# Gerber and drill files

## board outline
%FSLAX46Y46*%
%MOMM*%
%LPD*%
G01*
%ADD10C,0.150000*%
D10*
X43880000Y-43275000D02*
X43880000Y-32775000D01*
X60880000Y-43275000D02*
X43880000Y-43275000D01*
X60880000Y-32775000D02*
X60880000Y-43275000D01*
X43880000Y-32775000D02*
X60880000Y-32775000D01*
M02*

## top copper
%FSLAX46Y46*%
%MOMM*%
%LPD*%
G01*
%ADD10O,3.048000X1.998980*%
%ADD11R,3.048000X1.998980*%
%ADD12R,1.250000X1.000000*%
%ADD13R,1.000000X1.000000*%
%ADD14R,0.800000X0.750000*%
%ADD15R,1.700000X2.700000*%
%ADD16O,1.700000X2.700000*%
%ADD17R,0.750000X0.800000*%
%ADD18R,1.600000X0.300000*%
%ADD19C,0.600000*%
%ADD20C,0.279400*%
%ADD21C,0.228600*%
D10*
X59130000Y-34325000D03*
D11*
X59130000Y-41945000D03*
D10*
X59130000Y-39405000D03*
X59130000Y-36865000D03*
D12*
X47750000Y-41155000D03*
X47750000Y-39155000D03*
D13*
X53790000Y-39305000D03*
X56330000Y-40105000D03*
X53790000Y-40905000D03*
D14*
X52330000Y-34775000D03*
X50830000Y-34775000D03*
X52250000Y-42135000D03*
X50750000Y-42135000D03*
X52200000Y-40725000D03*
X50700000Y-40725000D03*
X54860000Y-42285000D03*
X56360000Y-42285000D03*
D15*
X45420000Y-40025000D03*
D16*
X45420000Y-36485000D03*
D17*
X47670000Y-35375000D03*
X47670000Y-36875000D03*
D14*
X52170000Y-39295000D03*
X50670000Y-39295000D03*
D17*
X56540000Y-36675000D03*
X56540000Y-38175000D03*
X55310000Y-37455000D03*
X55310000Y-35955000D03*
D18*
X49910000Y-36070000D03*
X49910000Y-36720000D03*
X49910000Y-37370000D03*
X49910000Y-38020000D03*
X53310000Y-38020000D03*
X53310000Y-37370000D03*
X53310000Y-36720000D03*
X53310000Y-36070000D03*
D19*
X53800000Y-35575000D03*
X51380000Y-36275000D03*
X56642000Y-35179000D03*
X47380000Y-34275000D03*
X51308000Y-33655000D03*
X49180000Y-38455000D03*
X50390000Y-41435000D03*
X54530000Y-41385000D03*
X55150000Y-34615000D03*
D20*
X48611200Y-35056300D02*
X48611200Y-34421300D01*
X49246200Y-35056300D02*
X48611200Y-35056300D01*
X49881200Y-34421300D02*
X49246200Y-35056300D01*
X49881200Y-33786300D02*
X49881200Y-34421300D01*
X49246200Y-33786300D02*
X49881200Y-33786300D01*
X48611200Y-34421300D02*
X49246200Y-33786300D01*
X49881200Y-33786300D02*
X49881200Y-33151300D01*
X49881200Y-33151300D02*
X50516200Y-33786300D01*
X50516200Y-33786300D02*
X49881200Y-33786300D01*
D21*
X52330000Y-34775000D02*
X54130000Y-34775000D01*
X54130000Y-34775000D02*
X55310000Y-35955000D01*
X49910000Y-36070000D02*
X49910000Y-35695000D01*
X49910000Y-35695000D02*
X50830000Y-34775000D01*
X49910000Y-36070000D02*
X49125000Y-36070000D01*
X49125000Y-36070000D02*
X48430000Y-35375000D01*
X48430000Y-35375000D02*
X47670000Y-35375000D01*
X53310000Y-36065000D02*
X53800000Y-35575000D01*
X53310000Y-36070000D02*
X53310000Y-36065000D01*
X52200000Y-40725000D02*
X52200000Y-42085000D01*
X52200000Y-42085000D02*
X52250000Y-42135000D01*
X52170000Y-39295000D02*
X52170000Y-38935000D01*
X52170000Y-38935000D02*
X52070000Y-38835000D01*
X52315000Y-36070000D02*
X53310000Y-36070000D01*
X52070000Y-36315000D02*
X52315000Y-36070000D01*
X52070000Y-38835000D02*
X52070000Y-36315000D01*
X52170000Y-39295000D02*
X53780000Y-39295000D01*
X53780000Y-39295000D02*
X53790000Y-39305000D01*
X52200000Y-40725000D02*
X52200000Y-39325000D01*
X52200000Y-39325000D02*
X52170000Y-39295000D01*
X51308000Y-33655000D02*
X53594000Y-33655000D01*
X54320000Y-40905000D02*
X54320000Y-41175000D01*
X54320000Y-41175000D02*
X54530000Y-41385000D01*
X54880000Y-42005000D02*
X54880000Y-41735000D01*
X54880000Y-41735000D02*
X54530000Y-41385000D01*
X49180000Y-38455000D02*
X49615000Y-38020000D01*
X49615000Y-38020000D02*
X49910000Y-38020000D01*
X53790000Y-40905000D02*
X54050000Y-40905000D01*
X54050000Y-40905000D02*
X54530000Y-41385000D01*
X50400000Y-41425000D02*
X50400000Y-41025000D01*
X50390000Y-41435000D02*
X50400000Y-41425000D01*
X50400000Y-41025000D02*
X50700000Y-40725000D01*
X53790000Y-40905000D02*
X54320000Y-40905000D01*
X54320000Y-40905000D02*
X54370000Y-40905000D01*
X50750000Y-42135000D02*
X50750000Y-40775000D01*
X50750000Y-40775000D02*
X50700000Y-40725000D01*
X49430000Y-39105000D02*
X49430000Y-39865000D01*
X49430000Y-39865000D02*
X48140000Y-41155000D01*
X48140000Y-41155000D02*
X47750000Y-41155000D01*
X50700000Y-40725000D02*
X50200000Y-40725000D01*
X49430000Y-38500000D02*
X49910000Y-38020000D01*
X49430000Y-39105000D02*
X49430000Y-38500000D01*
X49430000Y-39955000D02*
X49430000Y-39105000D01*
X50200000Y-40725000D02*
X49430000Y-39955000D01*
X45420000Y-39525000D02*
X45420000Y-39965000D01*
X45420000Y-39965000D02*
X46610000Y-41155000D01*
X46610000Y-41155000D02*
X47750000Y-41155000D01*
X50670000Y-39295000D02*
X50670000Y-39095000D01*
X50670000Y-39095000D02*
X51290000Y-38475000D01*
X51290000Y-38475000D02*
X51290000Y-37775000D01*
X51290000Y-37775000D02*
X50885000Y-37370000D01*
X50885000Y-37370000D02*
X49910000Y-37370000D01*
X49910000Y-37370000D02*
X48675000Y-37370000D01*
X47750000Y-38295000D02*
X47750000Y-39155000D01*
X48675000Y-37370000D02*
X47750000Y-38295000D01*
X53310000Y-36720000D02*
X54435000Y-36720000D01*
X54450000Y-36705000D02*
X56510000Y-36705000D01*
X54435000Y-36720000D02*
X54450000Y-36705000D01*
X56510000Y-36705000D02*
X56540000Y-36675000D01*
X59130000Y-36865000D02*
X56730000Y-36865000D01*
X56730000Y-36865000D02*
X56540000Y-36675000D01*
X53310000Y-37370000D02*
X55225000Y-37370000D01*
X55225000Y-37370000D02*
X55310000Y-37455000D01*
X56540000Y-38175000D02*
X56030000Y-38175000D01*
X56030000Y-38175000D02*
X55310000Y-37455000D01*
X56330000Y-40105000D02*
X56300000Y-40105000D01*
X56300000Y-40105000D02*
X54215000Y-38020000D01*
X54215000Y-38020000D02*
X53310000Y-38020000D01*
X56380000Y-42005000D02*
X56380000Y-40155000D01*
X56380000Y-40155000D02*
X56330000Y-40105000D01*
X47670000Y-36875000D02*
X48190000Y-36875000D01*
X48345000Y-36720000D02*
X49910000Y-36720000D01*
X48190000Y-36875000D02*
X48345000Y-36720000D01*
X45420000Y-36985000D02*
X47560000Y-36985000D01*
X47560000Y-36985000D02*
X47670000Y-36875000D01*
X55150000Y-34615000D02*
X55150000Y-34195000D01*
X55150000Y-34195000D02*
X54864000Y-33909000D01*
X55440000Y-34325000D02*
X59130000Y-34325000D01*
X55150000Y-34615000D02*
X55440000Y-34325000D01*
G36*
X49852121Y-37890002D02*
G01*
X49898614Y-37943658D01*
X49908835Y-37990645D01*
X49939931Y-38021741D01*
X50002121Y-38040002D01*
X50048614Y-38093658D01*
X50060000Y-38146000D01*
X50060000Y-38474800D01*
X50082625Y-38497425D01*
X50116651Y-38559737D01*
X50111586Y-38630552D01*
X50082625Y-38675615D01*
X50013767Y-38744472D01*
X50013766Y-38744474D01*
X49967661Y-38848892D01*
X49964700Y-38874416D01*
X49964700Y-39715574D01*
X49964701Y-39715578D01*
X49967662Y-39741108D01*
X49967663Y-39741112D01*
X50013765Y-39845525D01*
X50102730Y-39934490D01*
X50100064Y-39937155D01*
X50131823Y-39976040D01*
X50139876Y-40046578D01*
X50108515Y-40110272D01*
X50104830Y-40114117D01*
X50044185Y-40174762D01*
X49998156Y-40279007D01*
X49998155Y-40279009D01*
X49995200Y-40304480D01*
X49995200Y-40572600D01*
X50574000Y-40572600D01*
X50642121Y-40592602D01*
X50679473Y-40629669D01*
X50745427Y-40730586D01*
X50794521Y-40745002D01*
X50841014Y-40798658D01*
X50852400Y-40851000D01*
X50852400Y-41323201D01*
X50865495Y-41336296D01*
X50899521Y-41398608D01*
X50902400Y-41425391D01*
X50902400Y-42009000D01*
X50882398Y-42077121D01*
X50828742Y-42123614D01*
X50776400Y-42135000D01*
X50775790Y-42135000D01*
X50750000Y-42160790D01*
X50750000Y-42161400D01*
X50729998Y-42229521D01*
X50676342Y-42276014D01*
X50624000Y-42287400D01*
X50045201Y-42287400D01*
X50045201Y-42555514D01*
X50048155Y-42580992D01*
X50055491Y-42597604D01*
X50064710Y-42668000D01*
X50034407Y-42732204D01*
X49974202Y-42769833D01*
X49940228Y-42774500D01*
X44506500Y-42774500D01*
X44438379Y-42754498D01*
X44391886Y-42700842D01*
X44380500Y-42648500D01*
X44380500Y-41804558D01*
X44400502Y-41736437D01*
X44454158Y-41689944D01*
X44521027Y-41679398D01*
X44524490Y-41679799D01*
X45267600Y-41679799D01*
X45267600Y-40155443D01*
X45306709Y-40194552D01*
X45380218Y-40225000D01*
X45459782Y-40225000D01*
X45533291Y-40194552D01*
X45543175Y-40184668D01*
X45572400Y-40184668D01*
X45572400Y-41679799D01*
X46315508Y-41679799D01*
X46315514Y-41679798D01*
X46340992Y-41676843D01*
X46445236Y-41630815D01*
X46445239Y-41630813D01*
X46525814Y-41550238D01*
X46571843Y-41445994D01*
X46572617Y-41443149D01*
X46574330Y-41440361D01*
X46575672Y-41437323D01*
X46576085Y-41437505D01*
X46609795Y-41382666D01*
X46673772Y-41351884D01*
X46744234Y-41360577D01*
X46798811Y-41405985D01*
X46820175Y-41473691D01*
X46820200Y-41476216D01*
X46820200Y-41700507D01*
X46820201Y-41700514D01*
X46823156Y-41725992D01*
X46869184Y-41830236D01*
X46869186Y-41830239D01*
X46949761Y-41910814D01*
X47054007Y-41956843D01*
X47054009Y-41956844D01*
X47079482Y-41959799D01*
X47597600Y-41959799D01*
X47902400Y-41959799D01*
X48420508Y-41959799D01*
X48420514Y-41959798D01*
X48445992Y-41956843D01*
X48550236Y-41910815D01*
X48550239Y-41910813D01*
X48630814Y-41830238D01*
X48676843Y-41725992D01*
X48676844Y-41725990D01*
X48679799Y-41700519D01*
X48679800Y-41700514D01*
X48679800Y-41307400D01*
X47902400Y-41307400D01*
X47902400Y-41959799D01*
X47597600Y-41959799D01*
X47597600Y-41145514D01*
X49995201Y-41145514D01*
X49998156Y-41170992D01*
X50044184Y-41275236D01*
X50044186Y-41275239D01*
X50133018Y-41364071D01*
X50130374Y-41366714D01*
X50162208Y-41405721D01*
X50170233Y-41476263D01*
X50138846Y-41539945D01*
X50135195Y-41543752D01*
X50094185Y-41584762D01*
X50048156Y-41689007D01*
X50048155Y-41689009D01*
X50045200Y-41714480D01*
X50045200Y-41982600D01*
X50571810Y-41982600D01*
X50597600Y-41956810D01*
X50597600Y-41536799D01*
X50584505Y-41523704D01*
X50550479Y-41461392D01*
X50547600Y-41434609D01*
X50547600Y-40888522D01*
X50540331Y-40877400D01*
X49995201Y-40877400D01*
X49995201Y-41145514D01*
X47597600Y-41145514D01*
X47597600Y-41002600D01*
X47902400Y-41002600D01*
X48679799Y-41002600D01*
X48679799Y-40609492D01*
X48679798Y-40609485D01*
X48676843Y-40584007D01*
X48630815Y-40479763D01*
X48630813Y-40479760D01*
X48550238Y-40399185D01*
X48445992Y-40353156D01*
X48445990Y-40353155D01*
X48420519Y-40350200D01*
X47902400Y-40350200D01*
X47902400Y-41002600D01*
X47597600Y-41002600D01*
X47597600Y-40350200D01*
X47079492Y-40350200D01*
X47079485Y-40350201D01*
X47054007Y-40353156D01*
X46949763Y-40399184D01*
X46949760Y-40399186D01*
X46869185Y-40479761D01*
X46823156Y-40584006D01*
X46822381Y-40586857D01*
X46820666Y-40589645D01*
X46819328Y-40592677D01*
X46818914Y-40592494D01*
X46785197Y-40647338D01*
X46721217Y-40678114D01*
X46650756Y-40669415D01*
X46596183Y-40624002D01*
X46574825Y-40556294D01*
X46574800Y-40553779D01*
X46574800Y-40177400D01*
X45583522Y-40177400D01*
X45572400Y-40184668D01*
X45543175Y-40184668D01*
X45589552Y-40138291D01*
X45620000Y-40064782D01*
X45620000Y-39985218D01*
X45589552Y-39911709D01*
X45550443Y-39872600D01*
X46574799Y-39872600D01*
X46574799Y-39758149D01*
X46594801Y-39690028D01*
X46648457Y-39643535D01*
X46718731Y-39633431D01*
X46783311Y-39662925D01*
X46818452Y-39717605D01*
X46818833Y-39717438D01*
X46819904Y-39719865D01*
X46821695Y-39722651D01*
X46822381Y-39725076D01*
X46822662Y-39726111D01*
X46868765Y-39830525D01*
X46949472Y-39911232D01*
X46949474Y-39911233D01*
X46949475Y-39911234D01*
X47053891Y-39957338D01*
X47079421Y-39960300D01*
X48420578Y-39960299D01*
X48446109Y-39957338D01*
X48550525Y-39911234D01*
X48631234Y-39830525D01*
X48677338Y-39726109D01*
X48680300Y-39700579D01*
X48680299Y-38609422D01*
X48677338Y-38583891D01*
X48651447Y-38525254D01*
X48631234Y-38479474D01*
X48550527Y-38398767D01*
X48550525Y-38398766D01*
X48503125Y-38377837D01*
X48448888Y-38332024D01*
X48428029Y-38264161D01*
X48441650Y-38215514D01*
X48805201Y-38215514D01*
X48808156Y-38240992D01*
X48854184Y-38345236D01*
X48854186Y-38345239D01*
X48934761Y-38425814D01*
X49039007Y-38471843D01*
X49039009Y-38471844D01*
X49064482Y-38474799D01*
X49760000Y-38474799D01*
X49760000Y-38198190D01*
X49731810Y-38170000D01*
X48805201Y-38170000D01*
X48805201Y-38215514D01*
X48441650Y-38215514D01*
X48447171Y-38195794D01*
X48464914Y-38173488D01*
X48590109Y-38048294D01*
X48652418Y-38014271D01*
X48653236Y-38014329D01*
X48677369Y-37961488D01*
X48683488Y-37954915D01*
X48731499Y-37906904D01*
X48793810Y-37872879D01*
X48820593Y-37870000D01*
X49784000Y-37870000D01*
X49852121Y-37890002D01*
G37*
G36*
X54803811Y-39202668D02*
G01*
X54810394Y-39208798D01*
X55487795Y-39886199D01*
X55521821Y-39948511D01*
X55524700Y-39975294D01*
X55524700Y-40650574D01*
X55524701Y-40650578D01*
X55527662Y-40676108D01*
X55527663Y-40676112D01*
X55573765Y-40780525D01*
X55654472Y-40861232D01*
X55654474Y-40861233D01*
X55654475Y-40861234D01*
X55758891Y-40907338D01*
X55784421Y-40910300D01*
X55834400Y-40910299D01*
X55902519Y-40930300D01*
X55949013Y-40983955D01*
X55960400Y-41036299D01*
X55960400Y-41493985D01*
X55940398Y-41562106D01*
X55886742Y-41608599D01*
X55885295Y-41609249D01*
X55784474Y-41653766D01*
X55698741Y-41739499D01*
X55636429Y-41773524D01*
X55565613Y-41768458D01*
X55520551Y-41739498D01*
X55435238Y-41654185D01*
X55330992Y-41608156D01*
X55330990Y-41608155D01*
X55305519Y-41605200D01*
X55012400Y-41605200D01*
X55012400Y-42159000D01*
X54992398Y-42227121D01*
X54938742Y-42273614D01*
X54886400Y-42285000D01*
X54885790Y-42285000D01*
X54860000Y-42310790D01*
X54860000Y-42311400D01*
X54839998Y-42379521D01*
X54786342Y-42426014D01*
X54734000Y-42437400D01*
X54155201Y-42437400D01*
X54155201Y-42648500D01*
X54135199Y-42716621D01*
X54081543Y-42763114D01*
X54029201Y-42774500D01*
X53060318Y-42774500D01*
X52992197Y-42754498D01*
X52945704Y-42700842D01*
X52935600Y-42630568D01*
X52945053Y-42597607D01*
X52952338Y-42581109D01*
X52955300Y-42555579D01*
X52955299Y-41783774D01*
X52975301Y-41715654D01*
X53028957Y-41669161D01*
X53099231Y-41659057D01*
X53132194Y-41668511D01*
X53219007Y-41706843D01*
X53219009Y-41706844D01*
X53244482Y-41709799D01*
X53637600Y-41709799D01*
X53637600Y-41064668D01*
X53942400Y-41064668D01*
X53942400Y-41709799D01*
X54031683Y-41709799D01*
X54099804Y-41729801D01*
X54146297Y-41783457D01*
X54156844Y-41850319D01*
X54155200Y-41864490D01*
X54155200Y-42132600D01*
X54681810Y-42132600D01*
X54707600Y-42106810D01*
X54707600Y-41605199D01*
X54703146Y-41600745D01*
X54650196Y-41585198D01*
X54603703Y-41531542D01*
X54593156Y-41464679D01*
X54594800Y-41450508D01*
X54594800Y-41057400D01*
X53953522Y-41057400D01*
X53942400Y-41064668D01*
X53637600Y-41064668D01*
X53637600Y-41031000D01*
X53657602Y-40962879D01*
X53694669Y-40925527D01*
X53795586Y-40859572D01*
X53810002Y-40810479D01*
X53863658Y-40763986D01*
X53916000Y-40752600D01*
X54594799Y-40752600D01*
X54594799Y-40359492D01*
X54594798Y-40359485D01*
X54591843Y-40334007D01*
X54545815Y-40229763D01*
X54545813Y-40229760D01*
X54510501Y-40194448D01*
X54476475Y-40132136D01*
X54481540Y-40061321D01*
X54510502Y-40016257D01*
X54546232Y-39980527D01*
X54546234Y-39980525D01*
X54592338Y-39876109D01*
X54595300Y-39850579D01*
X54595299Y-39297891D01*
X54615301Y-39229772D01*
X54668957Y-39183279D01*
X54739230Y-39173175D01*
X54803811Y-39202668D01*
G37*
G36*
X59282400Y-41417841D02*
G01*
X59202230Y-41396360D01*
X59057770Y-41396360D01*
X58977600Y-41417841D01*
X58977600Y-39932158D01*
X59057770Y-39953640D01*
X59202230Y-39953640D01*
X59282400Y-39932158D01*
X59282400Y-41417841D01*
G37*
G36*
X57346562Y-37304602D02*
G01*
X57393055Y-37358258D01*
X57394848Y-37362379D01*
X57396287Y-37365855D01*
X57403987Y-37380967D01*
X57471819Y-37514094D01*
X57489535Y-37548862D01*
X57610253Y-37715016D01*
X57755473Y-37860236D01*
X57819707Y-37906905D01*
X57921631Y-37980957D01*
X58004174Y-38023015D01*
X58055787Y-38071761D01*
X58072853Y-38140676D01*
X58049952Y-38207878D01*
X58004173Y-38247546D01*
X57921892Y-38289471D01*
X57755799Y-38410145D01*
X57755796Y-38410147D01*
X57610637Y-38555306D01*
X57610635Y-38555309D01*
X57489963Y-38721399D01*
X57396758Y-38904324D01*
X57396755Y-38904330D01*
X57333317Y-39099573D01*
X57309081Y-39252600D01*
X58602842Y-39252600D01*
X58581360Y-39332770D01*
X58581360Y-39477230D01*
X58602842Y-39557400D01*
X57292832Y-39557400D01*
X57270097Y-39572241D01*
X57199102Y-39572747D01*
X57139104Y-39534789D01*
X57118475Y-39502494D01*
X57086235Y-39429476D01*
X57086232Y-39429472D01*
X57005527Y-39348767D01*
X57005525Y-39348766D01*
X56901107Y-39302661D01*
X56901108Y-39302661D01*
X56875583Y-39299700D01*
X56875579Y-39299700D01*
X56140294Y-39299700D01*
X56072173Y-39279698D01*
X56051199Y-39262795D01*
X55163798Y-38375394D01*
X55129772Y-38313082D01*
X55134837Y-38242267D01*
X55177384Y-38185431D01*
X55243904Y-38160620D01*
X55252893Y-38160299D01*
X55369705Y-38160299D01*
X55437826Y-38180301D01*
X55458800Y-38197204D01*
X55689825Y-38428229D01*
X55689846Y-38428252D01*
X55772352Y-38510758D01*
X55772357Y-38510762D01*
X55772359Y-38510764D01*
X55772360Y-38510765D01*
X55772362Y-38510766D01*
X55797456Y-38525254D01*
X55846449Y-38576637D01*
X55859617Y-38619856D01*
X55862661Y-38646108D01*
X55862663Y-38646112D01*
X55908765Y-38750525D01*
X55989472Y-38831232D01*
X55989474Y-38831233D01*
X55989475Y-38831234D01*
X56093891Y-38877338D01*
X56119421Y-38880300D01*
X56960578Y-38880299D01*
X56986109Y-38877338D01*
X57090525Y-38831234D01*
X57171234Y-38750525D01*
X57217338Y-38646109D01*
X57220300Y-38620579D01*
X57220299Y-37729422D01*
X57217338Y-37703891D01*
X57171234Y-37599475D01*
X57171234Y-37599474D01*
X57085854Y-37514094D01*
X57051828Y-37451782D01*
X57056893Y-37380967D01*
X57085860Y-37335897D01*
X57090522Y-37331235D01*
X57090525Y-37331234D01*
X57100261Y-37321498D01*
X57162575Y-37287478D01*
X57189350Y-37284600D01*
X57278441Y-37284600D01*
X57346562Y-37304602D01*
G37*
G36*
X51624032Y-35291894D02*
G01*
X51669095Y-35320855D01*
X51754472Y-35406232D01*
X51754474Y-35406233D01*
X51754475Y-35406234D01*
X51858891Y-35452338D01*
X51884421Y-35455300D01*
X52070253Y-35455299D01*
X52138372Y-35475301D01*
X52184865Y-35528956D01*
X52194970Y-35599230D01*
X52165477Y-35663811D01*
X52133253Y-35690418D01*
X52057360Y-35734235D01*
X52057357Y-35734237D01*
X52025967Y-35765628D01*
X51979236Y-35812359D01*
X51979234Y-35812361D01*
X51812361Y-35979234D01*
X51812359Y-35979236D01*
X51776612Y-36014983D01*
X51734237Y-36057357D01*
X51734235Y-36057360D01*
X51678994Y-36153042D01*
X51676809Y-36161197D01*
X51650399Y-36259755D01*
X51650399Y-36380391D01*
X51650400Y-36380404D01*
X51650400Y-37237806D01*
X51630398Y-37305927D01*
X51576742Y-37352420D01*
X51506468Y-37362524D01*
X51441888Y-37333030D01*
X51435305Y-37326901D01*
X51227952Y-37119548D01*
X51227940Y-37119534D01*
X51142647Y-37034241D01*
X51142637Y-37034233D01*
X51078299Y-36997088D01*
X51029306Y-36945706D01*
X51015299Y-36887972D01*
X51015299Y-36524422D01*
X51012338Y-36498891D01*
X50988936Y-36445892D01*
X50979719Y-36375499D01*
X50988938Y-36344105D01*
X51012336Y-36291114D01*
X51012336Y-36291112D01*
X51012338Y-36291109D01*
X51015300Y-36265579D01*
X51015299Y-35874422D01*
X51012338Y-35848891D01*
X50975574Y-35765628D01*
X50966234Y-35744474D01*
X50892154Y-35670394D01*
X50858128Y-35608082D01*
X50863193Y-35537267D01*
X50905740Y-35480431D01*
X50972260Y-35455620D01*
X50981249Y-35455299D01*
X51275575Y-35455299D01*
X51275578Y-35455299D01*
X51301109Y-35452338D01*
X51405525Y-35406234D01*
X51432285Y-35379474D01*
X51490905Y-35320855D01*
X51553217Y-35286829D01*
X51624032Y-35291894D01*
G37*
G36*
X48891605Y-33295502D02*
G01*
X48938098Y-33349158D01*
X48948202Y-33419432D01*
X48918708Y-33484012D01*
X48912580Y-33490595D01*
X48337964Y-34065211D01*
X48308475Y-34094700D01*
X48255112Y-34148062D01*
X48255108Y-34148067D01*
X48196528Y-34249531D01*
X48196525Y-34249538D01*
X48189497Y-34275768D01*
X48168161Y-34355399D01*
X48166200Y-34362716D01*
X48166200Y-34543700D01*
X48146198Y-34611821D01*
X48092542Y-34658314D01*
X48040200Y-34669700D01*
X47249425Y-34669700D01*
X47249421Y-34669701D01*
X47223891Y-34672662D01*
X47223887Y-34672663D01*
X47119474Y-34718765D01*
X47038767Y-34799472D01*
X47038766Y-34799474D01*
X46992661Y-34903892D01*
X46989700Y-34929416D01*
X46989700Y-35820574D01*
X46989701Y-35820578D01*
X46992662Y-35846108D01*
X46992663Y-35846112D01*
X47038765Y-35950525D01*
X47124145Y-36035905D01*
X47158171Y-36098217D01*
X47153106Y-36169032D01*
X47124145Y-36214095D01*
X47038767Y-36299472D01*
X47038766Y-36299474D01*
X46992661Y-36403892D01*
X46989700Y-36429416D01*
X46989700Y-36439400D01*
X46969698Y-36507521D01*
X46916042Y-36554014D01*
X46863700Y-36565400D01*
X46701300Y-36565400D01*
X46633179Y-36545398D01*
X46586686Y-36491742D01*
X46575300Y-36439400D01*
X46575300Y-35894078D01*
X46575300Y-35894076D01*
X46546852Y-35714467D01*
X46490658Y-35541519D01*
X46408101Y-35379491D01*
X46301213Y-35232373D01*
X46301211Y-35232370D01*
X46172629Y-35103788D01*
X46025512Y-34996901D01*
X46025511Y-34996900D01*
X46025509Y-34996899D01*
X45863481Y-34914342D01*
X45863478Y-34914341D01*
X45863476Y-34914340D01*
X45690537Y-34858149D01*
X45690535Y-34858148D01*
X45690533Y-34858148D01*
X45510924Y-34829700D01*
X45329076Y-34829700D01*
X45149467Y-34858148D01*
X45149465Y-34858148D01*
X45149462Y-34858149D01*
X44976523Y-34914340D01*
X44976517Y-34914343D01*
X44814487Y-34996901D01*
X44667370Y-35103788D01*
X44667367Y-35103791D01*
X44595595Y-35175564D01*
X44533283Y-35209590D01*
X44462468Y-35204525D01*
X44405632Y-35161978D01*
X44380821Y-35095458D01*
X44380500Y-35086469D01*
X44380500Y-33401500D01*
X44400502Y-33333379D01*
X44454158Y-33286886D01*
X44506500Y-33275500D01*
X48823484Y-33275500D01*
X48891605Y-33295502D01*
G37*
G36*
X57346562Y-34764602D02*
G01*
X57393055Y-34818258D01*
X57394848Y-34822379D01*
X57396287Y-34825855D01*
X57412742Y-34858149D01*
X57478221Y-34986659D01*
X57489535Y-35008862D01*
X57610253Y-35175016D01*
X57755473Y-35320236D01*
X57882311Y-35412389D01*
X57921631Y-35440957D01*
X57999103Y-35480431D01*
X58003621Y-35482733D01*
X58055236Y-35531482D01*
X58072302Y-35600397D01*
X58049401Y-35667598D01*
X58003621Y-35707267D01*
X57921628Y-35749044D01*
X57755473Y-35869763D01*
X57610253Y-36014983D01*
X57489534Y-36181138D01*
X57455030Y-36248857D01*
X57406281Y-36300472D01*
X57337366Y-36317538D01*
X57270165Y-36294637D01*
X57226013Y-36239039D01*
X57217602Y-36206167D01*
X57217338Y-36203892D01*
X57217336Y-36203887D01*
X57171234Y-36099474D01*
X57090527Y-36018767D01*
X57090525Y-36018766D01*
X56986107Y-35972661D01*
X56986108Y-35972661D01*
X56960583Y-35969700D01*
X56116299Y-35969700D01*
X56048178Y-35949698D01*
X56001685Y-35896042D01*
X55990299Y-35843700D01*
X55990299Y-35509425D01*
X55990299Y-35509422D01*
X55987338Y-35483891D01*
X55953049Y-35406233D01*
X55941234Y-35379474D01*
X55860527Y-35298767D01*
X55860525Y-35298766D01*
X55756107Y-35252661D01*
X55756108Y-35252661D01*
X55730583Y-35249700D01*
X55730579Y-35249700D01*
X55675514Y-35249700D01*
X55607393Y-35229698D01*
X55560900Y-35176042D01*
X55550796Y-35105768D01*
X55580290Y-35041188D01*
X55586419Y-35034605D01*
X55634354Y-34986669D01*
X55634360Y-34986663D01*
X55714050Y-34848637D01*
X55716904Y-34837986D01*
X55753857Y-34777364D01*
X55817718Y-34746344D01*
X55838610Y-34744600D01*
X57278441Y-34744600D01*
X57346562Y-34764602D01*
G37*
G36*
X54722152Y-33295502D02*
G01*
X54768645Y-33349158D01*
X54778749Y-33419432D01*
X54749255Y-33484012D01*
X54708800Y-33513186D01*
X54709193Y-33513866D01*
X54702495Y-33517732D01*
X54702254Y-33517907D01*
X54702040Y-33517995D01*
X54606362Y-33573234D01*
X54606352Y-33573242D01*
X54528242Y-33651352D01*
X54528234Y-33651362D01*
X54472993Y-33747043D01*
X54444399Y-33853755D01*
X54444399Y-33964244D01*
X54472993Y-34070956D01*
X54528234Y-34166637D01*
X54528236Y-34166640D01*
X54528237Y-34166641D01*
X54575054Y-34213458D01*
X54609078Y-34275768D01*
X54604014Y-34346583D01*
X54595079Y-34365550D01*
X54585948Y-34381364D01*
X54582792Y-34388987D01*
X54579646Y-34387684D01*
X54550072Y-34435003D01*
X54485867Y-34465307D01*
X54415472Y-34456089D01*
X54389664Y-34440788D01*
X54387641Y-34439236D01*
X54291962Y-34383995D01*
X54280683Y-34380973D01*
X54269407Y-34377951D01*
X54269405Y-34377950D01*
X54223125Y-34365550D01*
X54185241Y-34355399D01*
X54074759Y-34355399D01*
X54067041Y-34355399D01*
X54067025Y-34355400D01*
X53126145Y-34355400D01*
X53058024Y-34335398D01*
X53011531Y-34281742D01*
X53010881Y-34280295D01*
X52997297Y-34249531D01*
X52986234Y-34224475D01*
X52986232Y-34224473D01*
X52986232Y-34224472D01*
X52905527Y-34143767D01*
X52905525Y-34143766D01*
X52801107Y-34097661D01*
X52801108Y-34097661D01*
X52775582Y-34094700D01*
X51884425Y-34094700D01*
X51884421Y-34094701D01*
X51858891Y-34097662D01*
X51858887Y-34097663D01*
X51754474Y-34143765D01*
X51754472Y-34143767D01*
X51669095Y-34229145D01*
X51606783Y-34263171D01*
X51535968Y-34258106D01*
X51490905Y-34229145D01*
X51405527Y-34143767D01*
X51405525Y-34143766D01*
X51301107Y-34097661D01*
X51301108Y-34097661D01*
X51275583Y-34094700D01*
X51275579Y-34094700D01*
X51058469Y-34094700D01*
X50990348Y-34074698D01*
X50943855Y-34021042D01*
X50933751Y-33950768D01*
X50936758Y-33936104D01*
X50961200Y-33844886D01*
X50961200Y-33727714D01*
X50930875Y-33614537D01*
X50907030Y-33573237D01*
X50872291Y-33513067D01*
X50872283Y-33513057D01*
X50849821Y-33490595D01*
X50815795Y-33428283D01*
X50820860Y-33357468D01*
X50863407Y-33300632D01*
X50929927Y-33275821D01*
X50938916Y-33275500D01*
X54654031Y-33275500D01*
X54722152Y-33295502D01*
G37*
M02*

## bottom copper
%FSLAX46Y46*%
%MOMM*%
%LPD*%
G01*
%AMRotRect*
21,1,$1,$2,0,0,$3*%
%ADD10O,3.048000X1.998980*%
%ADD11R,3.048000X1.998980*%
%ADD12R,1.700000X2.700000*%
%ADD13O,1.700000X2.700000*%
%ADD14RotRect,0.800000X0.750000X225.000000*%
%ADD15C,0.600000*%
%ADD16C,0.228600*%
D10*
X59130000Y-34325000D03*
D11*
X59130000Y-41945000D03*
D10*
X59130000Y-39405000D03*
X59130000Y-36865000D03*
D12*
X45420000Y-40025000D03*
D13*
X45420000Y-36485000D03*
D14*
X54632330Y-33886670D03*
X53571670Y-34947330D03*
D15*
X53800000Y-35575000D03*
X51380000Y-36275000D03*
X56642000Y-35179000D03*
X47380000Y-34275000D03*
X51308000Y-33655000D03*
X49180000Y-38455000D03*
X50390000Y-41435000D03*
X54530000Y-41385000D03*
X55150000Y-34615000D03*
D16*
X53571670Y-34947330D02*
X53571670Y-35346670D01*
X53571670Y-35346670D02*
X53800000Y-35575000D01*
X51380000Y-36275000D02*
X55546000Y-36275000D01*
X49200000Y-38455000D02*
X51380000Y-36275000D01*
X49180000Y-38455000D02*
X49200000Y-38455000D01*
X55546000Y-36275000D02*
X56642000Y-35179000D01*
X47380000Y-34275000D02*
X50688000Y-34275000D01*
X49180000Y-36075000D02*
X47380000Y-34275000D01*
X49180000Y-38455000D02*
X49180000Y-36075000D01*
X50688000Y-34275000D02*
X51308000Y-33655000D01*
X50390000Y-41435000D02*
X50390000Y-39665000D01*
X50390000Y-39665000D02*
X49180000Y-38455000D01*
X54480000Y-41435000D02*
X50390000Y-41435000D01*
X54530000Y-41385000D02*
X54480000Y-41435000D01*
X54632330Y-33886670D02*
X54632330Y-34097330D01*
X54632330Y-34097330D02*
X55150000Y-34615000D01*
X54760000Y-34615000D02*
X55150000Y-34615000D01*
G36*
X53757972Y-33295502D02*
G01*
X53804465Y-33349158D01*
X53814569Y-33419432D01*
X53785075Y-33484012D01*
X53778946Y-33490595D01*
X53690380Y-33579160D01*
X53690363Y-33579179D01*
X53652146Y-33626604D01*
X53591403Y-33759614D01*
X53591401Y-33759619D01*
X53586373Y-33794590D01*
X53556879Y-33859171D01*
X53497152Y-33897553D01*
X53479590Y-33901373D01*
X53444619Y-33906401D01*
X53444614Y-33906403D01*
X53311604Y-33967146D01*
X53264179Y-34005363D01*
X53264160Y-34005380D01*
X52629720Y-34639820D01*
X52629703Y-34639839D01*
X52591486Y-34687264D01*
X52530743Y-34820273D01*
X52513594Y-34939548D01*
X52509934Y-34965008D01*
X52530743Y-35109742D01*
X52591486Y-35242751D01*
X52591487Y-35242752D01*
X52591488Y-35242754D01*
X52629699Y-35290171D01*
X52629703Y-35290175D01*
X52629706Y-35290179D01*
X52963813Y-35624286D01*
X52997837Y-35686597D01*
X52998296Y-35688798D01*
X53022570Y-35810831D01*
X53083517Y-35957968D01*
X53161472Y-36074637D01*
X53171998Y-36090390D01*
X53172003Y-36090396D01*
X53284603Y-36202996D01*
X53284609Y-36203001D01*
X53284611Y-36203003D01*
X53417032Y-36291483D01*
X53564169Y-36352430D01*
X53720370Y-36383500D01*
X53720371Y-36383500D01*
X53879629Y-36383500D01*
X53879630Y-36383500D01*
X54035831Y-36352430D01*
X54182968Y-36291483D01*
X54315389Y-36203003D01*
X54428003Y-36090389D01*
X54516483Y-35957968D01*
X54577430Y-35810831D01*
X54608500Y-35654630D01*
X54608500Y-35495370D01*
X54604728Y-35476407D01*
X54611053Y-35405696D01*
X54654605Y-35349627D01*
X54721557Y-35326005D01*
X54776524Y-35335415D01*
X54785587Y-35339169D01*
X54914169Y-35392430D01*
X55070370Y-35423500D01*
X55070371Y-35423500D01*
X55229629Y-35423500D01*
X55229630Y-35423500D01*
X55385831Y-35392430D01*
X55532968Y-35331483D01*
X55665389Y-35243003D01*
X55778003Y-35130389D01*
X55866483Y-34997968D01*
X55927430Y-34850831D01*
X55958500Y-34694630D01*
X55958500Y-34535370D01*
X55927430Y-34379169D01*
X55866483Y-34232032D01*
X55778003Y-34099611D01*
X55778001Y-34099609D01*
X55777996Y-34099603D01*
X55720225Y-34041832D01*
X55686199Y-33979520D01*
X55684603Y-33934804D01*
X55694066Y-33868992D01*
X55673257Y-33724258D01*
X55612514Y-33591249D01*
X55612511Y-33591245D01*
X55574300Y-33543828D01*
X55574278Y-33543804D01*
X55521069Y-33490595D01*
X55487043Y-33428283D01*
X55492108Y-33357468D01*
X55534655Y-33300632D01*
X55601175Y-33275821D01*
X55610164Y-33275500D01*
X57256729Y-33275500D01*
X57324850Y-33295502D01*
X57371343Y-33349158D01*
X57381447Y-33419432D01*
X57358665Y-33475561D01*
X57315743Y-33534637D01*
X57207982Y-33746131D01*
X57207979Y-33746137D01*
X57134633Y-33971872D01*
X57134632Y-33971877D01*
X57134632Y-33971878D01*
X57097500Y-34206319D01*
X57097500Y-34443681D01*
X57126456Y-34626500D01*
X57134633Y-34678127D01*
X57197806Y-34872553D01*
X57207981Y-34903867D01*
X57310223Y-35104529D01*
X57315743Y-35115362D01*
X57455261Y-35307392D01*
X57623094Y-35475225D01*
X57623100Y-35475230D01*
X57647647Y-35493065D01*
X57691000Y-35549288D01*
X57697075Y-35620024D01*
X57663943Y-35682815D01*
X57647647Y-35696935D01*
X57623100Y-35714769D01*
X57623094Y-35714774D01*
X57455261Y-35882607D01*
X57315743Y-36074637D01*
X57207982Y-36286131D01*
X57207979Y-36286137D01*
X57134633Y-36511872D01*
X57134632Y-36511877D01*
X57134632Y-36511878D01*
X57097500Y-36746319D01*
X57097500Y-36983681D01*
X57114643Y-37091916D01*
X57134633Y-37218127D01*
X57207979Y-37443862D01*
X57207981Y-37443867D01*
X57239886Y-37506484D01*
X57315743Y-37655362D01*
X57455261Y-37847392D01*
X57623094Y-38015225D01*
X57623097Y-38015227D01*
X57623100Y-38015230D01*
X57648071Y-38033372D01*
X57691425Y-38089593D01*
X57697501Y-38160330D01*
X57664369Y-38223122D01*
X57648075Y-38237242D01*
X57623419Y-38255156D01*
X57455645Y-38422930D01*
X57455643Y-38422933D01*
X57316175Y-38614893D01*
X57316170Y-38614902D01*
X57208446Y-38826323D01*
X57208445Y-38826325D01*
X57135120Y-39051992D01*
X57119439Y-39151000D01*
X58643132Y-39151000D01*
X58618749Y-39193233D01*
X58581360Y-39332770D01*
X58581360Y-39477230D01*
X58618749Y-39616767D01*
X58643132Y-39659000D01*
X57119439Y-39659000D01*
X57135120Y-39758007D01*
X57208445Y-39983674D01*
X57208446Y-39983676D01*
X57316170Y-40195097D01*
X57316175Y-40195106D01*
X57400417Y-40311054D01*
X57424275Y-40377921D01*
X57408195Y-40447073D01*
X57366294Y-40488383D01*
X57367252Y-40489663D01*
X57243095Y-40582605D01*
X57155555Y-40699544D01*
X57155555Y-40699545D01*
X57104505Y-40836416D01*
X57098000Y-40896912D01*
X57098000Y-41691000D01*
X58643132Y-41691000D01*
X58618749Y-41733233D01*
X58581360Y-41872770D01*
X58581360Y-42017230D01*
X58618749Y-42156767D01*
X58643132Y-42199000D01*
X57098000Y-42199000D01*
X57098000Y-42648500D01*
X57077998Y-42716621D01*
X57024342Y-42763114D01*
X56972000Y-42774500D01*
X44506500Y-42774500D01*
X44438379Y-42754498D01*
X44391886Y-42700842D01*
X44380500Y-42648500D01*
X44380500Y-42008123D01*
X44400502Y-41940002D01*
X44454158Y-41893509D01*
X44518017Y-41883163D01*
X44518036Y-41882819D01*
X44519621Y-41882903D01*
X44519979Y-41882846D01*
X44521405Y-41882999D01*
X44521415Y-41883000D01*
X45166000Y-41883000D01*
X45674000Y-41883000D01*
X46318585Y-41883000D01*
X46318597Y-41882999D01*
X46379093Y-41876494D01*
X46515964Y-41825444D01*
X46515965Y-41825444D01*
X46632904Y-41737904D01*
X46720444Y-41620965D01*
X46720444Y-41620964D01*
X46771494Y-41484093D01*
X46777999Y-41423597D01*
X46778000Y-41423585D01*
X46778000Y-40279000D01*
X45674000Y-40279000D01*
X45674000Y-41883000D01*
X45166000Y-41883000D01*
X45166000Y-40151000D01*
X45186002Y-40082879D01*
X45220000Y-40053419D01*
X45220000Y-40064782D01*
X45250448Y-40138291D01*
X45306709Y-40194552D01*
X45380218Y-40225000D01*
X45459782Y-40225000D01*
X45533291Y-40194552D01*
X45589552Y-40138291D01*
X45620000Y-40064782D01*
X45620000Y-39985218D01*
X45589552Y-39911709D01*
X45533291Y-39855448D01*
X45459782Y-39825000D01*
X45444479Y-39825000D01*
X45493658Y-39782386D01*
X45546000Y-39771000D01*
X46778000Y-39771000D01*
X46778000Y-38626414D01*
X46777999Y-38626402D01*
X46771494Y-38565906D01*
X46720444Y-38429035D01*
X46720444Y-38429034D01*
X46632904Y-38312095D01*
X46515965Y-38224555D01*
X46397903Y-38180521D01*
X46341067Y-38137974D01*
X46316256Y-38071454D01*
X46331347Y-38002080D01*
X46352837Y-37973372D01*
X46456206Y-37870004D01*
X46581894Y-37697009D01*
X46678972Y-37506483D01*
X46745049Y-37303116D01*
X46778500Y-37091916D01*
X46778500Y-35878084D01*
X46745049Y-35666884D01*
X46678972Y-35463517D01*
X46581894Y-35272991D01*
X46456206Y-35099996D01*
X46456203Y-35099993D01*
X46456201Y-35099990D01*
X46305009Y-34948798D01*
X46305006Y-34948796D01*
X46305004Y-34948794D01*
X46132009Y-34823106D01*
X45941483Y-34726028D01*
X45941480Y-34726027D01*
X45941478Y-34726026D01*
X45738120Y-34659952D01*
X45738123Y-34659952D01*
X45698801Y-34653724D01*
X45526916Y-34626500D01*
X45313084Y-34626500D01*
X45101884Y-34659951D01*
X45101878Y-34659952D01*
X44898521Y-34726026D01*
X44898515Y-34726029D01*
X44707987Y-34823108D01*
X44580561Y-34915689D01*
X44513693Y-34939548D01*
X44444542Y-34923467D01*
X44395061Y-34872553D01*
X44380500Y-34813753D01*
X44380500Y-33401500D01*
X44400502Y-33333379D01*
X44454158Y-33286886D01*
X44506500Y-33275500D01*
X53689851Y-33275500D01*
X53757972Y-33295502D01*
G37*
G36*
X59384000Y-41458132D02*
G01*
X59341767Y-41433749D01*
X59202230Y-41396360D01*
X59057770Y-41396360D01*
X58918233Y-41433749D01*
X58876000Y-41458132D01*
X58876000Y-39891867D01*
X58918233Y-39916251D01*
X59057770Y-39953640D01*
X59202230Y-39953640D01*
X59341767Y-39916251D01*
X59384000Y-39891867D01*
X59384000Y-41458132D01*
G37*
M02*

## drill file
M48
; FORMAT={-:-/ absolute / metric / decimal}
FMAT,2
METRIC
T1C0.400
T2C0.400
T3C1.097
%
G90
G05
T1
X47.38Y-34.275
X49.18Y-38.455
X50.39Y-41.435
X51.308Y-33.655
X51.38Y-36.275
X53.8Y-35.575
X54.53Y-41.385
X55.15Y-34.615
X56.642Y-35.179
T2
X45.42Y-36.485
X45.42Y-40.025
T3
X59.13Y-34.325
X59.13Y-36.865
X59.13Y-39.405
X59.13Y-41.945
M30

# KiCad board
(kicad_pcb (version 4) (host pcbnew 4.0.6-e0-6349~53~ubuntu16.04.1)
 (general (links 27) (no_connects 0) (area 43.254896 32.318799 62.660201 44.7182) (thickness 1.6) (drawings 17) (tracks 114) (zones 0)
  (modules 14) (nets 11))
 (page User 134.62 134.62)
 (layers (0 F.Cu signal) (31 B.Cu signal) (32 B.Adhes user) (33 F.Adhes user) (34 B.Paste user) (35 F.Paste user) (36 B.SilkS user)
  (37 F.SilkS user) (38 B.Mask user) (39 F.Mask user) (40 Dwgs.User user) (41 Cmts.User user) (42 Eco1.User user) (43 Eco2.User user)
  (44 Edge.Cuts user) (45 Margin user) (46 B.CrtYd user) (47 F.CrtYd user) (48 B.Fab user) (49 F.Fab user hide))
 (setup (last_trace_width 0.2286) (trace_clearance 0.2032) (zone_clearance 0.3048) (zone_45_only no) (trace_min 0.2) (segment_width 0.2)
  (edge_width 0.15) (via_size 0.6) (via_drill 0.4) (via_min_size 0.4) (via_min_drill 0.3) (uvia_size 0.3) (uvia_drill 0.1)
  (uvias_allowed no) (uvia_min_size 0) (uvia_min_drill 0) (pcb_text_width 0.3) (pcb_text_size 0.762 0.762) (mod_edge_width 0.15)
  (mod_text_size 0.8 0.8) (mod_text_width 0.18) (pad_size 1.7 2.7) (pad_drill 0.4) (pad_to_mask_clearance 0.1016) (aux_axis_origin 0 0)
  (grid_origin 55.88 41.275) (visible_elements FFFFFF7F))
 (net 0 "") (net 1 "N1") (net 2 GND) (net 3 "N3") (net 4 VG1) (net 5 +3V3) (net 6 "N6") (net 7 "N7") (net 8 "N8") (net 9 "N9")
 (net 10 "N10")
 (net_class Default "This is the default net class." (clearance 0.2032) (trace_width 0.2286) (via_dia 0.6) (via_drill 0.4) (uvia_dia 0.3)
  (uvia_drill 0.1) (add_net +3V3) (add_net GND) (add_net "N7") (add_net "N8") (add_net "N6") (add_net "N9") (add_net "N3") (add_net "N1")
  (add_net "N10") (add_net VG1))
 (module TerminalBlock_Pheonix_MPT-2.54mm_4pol (layer F.Cu) (at 59.13 41.945 90)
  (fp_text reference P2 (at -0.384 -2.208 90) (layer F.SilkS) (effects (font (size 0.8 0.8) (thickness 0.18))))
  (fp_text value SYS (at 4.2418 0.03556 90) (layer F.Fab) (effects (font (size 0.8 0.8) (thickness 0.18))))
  (pad 4 thru_hole oval (at 7.62 0 270) (size 1.99898 3.048) (drill 1.09728) (layers *.Cu *.Mask F.SilkS) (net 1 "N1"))
  (pad 1 thru_hole rect (at 0 0 270) (size 1.99898 3.048) (drill 1.09728) (layers *.Cu *.Mask F.SilkS) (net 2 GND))
  (pad 2 thru_hole oval (at 2.54 0 270) (size 1.99898 3.048) (drill 1.09728) (layers *.Cu *.Mask F.SilkS) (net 2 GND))
  (pad 3 thru_hole oval (at 5.08 0 270) (size 1.99898 3.048) (drill 1.09728) (layers *.Cu *.Mask F.SilkS) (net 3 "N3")))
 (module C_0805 (layer F.Cu) (at 47.75 40.155 90)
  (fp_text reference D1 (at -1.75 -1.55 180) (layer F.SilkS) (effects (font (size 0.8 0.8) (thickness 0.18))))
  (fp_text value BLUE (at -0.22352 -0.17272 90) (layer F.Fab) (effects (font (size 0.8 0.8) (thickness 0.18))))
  (pad 1 smd rect (at -1 0 90) (size 1 1.25) (layers F.Cu F.Paste F.Mask) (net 2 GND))
  (pad 2 smd rect (at 1 0 90) (size 1 1.25) (layers F.Cu F.Paste F.Mask) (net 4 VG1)))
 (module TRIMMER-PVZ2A (layer F.Cu) (at 53.79 40.105 270)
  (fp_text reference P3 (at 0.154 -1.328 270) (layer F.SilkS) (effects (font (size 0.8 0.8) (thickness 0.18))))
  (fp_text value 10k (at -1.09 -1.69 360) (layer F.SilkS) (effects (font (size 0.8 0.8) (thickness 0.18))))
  (pad 1 smd rect (at -0.8 0 270) (size 1 1) (layers F.Cu F.Paste F.Mask) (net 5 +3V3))
  (pad 2 smd rect (at 0 -2.54 270) (size 1 1) (layers F.Cu F.Paste F.Mask) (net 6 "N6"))
  (pad 3 smd rect (at 0.8 0 270) (size 1 1) (layers F.Cu F.Paste F.Mask) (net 2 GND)))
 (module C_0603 (layer F.Cu) (at 51.58 34.775 180)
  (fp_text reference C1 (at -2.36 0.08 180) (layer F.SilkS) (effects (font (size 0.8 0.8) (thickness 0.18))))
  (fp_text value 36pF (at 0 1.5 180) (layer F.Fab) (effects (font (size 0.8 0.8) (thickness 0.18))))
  (pad 1 smd rect (at -0.75 0 180) (size 0.8 0.75) (layers F.Cu F.Paste F.Mask) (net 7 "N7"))
  (pad 2 smd rect (at 0.75 0 180) (size 0.8 0.75) (layers F.Cu F.Paste F.Mask) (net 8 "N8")))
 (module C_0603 (layer F.Cu) (at 51.5 42.135 180)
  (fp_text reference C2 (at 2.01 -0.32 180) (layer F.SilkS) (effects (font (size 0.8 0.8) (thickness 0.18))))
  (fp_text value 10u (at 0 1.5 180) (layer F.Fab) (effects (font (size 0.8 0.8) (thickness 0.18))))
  (pad 1 smd rect (at -0.75 0 180) (size 0.8 0.75) (layers F.Cu F.Paste F.Mask) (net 5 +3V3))
  (pad 2 smd rect (at 0.75 0 180) (size 0.8 0.75) (layers F.Cu F.Paste F.Mask) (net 2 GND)))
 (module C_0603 (layer F.Cu) (at 51.45 40.725 180)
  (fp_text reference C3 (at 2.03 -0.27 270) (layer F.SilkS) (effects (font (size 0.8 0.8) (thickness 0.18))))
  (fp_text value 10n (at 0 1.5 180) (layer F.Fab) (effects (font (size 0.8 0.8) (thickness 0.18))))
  (pad 1 smd rect (at -0.75 0 180) (size 0.8 0.75) (layers F.Cu F.Paste F.Mask) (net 5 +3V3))
  (pad 2 smd rect (at 0.75 0 180) (size 0.8 0.75) (layers F.Cu F.Paste F.Mask) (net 2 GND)))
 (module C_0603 (layer F.Cu) (at 55.61 42.285)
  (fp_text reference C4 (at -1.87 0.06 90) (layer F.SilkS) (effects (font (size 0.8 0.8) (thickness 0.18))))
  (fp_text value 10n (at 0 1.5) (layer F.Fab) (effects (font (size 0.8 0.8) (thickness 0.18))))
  (pad 1 smd rect (at -0.75 0) (size 0.8 0.75) (layers F.Cu F.Paste F.Mask) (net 2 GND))
  (pad 2 smd rect (at 0.75 0) (size 0.8 0.75) (layers F.Cu F.Paste F.Mask) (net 6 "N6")))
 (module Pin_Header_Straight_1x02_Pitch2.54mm (layer F.Cu) (at 45.42 39.525 180)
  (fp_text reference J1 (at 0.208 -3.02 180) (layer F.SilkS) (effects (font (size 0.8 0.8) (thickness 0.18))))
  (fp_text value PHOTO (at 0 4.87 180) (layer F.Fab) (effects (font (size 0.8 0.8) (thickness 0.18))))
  (pad 1 thru_hole rect (at 0 -0.5 180) (size 1.7 2.7) (drill 0.4) (layers *.Cu *.Mask) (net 2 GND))
  (pad 2 thru_hole oval (at 0 3.04 180) (size 1.7 2.7) (drill 0.4) (layers *.Cu *.Mask) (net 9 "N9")))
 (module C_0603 (layer F.Cu) (at 47.67 36.125 270)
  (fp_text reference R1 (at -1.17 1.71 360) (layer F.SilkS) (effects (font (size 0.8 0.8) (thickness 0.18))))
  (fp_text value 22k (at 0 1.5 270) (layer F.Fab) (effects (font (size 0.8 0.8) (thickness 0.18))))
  (pad 1 smd rect (at -0.75 0 270) (size 0.8 0.75) (layers F.Cu F.Paste F.Mask) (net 8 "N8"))
  (pad 2 smd rect (at 0.75 0 270) (size 0.8 0.75) (layers F.Cu F.Paste F.Mask) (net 9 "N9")))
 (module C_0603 (layer F.Cu) (at 51.42 39.295 180)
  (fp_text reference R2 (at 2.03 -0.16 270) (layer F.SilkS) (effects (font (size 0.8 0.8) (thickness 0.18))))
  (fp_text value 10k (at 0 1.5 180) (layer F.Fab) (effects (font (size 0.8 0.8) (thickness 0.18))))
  (pad 1 smd rect (at -0.75 0 180) (size 0.8 0.75) (layers F.Cu F.Paste F.Mask) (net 5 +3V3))
  (pad 2 smd rect (at 0.75 0 180) (size 0.8 0.75) (layers F.Cu F.Paste F.Mask) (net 4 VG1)))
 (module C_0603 (layer F.Cu) (at 56.54 37.425 270)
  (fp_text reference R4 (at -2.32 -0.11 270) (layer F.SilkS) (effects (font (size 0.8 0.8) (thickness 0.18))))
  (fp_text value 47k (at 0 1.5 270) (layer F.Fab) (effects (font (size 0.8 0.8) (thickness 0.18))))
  (pad 1 smd rect (at -0.75 0 270) (size 0.8 0.75) (layers F.Cu F.Paste F.Mask) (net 3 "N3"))
  (pad 2 smd rect (at 0.75 0 270) (size 0.8 0.75) (layers F.Cu F.Paste F.Mask) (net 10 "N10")))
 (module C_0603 (layer F.Cu) (at 55.31 36.705 90)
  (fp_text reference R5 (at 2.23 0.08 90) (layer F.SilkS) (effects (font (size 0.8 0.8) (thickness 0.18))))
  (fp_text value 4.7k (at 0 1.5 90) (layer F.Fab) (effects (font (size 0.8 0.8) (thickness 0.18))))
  (pad 1 smd rect (at -0.75 0 90) (size 0.8 0.75) (layers F.Cu F.Paste F.Mask) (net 10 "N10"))
  (pad 2 smd rect (at 0.75 0 90) (size 0.8 0.75) (layers F.Cu F.Paste F.Mask) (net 7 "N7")))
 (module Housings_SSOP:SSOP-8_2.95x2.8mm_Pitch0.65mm (layer F.Cu) (at 51.61 37.045)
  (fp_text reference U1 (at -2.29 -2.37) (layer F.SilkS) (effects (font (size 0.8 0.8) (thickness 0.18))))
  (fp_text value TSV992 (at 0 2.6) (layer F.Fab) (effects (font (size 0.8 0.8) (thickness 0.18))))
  (pad 1 smd rect (at -1.7 -0.975 270) (size 0.3 1.6) (layers F.Cu F.Paste F.Mask) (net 8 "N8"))
  (pad 2 smd rect (at -1.7 -0.325 270) (size 0.3 1.6) (layers F.Cu F.Paste F.Mask) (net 9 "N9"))
  (pad 3 smd rect (at -1.7 0.325 270) (size 0.3 1.6) (layers F.Cu F.Paste F.Mask) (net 4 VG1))
  (pad 4 smd rect (at -1.7 0.975 270) (size 0.3 1.6) (layers F.Cu F.Paste F.Mask) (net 2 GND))
  (pad 5 smd rect (at 1.7 0.975 270) (size 0.3 1.6) (layers F.Cu F.Paste F.Mask) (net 6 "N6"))
  (pad 6 smd rect (at 1.7 0.325 270) (size 0.3 1.6) (layers F.Cu F.Paste F.Mask) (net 10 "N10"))
  (pad 7 smd rect (at 1.7 -0.325 270) (size 0.3 1.6) (layers F.Cu F.Paste F.Mask) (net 3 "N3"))
  (pad 8 smd rect (at 1.7 -0.975 270) (size 0.3 1.6) (layers F.Cu F.Paste F.Mask) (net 5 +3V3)))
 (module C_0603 (layer B.Cu) (at 54.102 34.417 225)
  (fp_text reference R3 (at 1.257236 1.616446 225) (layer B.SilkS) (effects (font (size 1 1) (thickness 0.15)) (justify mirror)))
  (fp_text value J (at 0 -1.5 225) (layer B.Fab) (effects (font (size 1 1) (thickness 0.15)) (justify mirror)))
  (pad 1 smd rect (at -0.75 0 225) (size 0.8 0.75) (layers B.Cu B.Paste B.Mask) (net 1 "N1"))
  (pad 2 smd rect (at 0.75 0 225) (size 0.8 0.75) (layers B.Cu B.Paste B.Mask) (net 5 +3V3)))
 (gr_line (start 43.88 43.275) (end 43.88 32.775) (angle 90) (layer Edge.Cuts) (width 0.15))
 (gr_line (start 60.88 43.275) (end 43.88 43.275) (angle 90) (layer Edge.Cuts) (width 0.15))
 (gr_line (start 60.88 32.775) (end 60.88 43.275) (angle 90) (layer Edge.Cuts) (width 0.15))
 (gr_line (start 43.88 32.775) (end 60.88 32.775) (angle 90) (layer Edge.Cuts) (width 0.15))
 (segment (start 48.6112 35.0563) (end 48.6112 34.4213) (width 0.2794) (layer F.Cu) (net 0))
 (segment (start 49.2462 35.0563) (end 48.6112 35.0563) (width 0.2794) (layer F.Cu) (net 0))
 (segment (start 49.8812 34.4213) (end 49.2462 35.0563) (width 0.2794) (layer F.Cu) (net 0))
 (segment (start 49.8812 33.7863) (end 49.8812 34.4213) (width 0.2794) (layer F.Cu) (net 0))
 (segment (start 49.2462 33.7863) (end 49.8812 33.7863) (width 0.2794) (layer F.Cu) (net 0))
 (segment (start 48.6112 34.4213) (end 49.2462 33.7863) (width 0.2794) (layer F.Cu) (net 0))
 (segment (start 49.8812 33.7863) (end 49.8812 33.1513) (width 0.2794) (layer F.Cu) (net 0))
 (segment (start 49.8812 33.1513) (end 50.5162 33.7863) (width 0.2794) (layer F.Cu) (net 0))
 (segment (start 50.5162 33.7863) (end 49.8812 33.7863) (width 0.2794) (layer F.Cu) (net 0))
 (segment (start 52.33 34.775) (end 54.13 34.775) (width 0.2286) (layer F.Cu) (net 7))
 (segment (start 54.13 34.775) (end 55.31 35.955) (width 0.2286) (layer F.Cu) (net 7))
 (segment (start 49.91 36.07) (end 49.91 35.695) (width 0.2286) (layer F.Cu) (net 8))
 (segment (start 49.91 35.695) (end 50.83 34.775) (width 0.2286) (layer F.Cu) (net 8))
 (segment (start 49.91 36.07) (end 49.125 36.07) (width 0.2286) (layer F.Cu) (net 8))
 (segment (start 49.125 36.07) (end 48.43 35.375) (width 0.2286) (layer F.Cu) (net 8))
 (segment (start 48.43 35.375) (end 47.67 35.375) (width 0.2286) (layer F.Cu) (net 8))
 (segment (start 53.57167 34.94733) (end 53.57167 35.34667) (width 0.2286) (layer B.Cu) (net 5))
 (segment (start 53.57167 35.34667) (end 53.8 35.575) (width 0.2286) (layer B.Cu) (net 5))
 (via (at 53.8 35.575) (size 0.6) (drill 0.4) (layers F.Cu B.Cu) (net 5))
 (segment (start 53.31 36.065) (end 53.8 35.575) (width 0.2286) (layer F.Cu) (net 5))
 (segment (start 53.31 36.07) (end 53.31 36.065) (width 0.2286) (layer F.Cu) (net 5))
 (segment (start 52.2 40.725) (end 52.2 42.085) (width 0.2286) (layer F.Cu) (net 5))
 (segment (start 52.2 42.085) (end 52.25 42.135) (width 0.2286) (layer F.Cu) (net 5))
 (segment (start 52.17 39.295) (end 52.17 38.935) (width 0.2286) (layer F.Cu) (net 5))
 (segment (start 52.17 38.935) (end 52.07 38.835) (width 0.2286) (layer F.Cu) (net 5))
 (segment (start 52.315 36.07) (end 53.31 36.07) (width 0.2286) (layer F.Cu) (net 5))
 (segment (start 52.07 36.315) (end 52.315 36.07) (width 0.2286) (layer F.Cu) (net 5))
 (segment (start 52.07 38.835) (end 52.07 36.315) (width 0.2286) (layer F.Cu) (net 5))
 (segment (start 52.17 39.295) (end 53.78 39.295) (width 0.2286) (layer F.Cu) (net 5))
 (segment (start 53.78 39.295) (end 53.79 39.305) (width 0.2286) (layer F.Cu) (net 5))
 (segment (start 52.2 40.725) (end 52.2 39.325) (width 0.2286) (layer F.Cu) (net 5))
 (segment (start 52.2 39.325) (end 52.17 39.295) (width 0.2286) (layer F.Cu) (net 5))
 (segment (start 51.38 36.275) (end 55.546 36.275) (width 0.2286) (layer B.Cu) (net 2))
 (segment (start 49.2 38.455) (end 51.38 36.275) (width 0.2286) (layer B.Cu) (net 2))
 (via (at 51.38 36.275) (size 0.6) (drill 0.4) (layers F.Cu B.Cu) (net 2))
 (segment (start 49.18 38.455) (end 49.2 38.455) (width 0.2286) (layer B.Cu) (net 2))
 (via (at 56.642 35.179) (size 0.6) (drill 0.4) (layers F.Cu B.Cu) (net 2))
 (segment (start 55.546 36.275) (end 56.642 35.179) (width 0.2286) (layer B.Cu) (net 2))
 (segment (start 47.38 34.275) (end 50.688 34.275) (width 0.2286) (layer B.Cu) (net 2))
 (segment (start 49.18 36.075) (end 47.38 34.275) (width 0.2286) (layer B.Cu) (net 2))
 (via (at 47.38 34.275) (size 0.6) (drill 0.4) (layers F.Cu B.Cu) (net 2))
 (segment (start 49.18 38.455) (end 49.18 36.075) (width 0.2286) (layer B.Cu) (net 2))
 (segment (start 51.308 33.655) (end 53.594 33.655) (width 0.2286) (layer F.Cu) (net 2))
 (via (at 51.308 33.655) (size 0.6) (drill 0.4) (layers F.Cu B.Cu) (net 2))
 (segment (start 50.688 34.275) (end 51.308 33.655) (width 0.2286) (layer B.Cu) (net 2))
 (segment (start 54.32 40.905) (end 54.32 41.175) (width 0.2286) (layer F.Cu) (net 2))
 (segment (start 54.32 41.175) (end 54.53 41.385) (width 0.2286) (layer F.Cu) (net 2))
 (segment (start 54.88 42.005) (end 54.88 41.735) (width 0.2286) (layer F.Cu) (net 2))
 (segment (start 54.88 41.735) (end 54.53 41.385) (width 0.2286) (layer F.Cu) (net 2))
 (segment (start 50.39 41.435) (end 50.39 39.665) (width 0.2286) (layer B.Cu) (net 2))
 (segment (start 49.18 38.455) (end 49.615 38.02) (width 0.2286) (layer F.Cu) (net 2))
 (via (at 49.18 38.455) (size 0.6) (drill 0.4) (layers F.Cu B.Cu) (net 2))
 (segment (start 50.39 39.665) (end 49.18 38.455) (width 0.2286) (layer B.Cu) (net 2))
 (segment (start 49.615 38.02) (end 49.91 38.02) (width 0.2286) (layer F.Cu) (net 2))
 (segment (start 53.79 40.905) (end 54.05 40.905) (width 0.2286) (layer F.Cu) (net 2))
 (segment (start 54.05 40.905) (end 54.53 41.385) (width 0.2286) (layer F.Cu) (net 2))
 (segment (start 50.4 41.425) (end 50.4 41.025) (width 0.2286) (layer F.Cu) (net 2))
 (segment (start 50.39 41.435) (end 50.4 41.425) (width 0.2286) (layer F.Cu) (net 2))
 (via (at 50.39 41.435) (size 0.6) (drill 0.4) (layers F.Cu B.Cu) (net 2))
 (segment (start 54.48 41.435) (end 50.39 41.435) (width 0.2286) (layer B.Cu) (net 2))
 (via (at 54.53 41.385) (size 0.6) (drill 0.4) (layers F.Cu B.Cu) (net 2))
 (segment (start 54.53 41.385) (end 54.48 41.435) (width 0.2286) (layer B.Cu) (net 2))
 (segment (start 50.4 41.025) (end 50.7 40.725) (width 0.2286) (layer F.Cu) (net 2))
 (segment (start 53.79 40.905) (end 54.32 40.905) (width 0.2286) (layer F.Cu) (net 2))
 (segment (start 54.32 40.905) (end 54.37 40.905) (width 0.2286) (layer F.Cu) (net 2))
 (segment (start 50.75 42.135) (end 50.75 40.775) (width 0.2286) (layer F.Cu) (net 2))
 (segment (start 50.75 40.775) (end 50.7 40.725) (width 0.2286) (layer F.Cu) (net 2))
 (segment (start 49.43 39.105) (end 49.43 39.865) (width 0.2286) (layer F.Cu) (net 2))
 (segment (start 49.43 39.865) (end 48.14 41.155) (width 0.2286) (layer F.Cu) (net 2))
 (segment (start 48.14 41.155) (end 47.75 41.155) (width 0.2286) (layer F.Cu) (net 2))
 (segment (start 50.7 40.725) (end 50.2 40.725) (width 0.2286) (layer F.Cu) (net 2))
 (segment (start 49.43 38.5) (end 49.91 38.02) (width 0.2286) (layer F.Cu) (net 2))
 (segment (start 49.43 39.105) (end 49.43 38.5) (width 0.2286) (layer F.Cu) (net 2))
 (segment (start 49.43 39.955) (end 49.43 39.105) (width 0.2286) (layer F.Cu) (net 2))
 (segment (start 50.2 40.725) (end 49.43 39.955) (width 0.2286) (layer F.Cu) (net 2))
 (segment (start 45.42 39.525) (end 45.42 39.965) (width 0.2286) (layer F.Cu) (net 2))
 (segment (start 45.42 39.965) (end 46.61 41.155) (width 0.2286) (layer F.Cu) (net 2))
 (segment (start 46.61 41.155) (end 47.75 41.155) (width 0.2286) (layer F.Cu) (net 2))
 (segment (start 50.67 39.295) (end 50.67 39.095) (width 0.2286) (layer F.Cu) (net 4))
 (segment (start 50.67 39.095) (end 51.29 38.475) (width 0.2286) (layer F.Cu) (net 4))
 (segment (start 51.29 38.475) (end 51.29 37.775) (width 0.2286) (layer F.Cu) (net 4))
 (segment (start 51.29 37.775) (end 50.885 37.37) (width 0.2286) (layer F.Cu) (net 4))
 (segment (start 50.885 37.37) (end 49.91 37.37) (width 0.2286) (layer F.Cu) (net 4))
 (segment (start 49.91 37.37) (end 48.675 37.37) (width 0.2286) (layer F.Cu) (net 4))
 (segment (start 47.75 38.295) (end 47.75 39.155) (width 0.2286) (layer F.Cu) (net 4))
 (segment (start 48.675 37.37) (end 47.75 38.295) (width 0.2286) (layer F.Cu) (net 4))
 (segment (start 53.31 36.72) (end 54.435 36.72) (width 0.2286) (layer F.Cu) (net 3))
 (segment (start 54.45 36.705) (end 56.51 36.705) (width 0.2286) (layer F.Cu) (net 3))
 (segment (start 54.435 36.72) (end 54.45 36.705) (width 0.2286) (layer F.Cu) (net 3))
 (segment (start 56.51 36.705) (end 56.54 36.675) (width 0.2286) (layer F.Cu) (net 3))
 (segment (start 59.13 36.865) (end 56.73 36.865) (width 0.2286) (layer F.Cu) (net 3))
 (segment (start 56.73 36.865) (end 56.54 36.675) (width 0.2286) (layer F.Cu) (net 3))
 (segment (start 53.31 37.37) (end 55.225 37.37) (width 0.2286) (layer F.Cu) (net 10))
 (segment (start 55.225 37.37) (end 55.31 37.455) (width 0.2286) (layer F.Cu) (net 10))
 (segment (start 56.54 38.175) (end 56.03 38.175) (width 0.2286) (layer F.Cu) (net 10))
 (segment (start 56.03 38.175) (end 55.31 37.455) (width 0.2286) (layer F.Cu) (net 10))
 (segment (start 56.33 40.105) (end 56.3 40.105) (width 0.2286) (layer F.Cu) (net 6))
 (segment (start 56.3 40.105) (end 54.215 38.02) (width 0.2286) (layer F.Cu) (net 6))
 (segment (start 54.215 38.02) (end 53.31 38.02) (width 0.2286) (layer F.Cu) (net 6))
 (segment (start 56.38 42.005) (end 56.38 40.155) (width 0.2286) (layer F.Cu) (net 6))
 (segment (start 56.38 40.155) (end 56.33 40.105) (width 0.2286) (layer F.Cu) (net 6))
 (segment (start 47.67 36.875) (end 48.19 36.875) (width 0.2286) (layer F.Cu) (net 9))
 (segment (start 48.345 36.72) (end 49.91 36.72) (width 0.2286) (layer F.Cu) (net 9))
 (segment (start 48.19 36.875) (end 48.345 36.72) (width 0.2286) (layer F.Cu) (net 9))
 (segment (start 45.42 36.985) (end 47.56 36.985) (width 0.2286) (layer F.Cu) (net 9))
 (segment (start 47.56 36.985) (end 47.67 36.875) (width 0.2286) (layer F.Cu) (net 9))
 (segment (start 54.63233 33.88667) (end 54.63233 34.09733) (width 0.2286) (layer B.Cu) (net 1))
 (segment (start 54.63233 34.09733) (end 55.15 34.615) (width 0.2286) (layer B.Cu) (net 1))
 (segment (start 55.15 34.615) (end 55.15 34.195) (width 0.2286) (layer F.Cu) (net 1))
 (segment (start 55.15 34.195) (end 54.864 33.909) (width 0.2286) (layer F.Cu) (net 1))
 (segment (start 55.44 34.325) (end 59.13 34.325) (width 0.2286) (layer F.Cu) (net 1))
 (segment (start 55.15 34.615) (end 55.44 34.325) (width 0.2286) (layer F.Cu) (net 1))
 (via (at 55.15 34.615) (size 0.6) (drill 0.4) (layers F.Cu B.Cu) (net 1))
 (segment (start 54.76 34.615) (end 55.15 34.615) (width 0.2286) (layer B.Cu) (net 1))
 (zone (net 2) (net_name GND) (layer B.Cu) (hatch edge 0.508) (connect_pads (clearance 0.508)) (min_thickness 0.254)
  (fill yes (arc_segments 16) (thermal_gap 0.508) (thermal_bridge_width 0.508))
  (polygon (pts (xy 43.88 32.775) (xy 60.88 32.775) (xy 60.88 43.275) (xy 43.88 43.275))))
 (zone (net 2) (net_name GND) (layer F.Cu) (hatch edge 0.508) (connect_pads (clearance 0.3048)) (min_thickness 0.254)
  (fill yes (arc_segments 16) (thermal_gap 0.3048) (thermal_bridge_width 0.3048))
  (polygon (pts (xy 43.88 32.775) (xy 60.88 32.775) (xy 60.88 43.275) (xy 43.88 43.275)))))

